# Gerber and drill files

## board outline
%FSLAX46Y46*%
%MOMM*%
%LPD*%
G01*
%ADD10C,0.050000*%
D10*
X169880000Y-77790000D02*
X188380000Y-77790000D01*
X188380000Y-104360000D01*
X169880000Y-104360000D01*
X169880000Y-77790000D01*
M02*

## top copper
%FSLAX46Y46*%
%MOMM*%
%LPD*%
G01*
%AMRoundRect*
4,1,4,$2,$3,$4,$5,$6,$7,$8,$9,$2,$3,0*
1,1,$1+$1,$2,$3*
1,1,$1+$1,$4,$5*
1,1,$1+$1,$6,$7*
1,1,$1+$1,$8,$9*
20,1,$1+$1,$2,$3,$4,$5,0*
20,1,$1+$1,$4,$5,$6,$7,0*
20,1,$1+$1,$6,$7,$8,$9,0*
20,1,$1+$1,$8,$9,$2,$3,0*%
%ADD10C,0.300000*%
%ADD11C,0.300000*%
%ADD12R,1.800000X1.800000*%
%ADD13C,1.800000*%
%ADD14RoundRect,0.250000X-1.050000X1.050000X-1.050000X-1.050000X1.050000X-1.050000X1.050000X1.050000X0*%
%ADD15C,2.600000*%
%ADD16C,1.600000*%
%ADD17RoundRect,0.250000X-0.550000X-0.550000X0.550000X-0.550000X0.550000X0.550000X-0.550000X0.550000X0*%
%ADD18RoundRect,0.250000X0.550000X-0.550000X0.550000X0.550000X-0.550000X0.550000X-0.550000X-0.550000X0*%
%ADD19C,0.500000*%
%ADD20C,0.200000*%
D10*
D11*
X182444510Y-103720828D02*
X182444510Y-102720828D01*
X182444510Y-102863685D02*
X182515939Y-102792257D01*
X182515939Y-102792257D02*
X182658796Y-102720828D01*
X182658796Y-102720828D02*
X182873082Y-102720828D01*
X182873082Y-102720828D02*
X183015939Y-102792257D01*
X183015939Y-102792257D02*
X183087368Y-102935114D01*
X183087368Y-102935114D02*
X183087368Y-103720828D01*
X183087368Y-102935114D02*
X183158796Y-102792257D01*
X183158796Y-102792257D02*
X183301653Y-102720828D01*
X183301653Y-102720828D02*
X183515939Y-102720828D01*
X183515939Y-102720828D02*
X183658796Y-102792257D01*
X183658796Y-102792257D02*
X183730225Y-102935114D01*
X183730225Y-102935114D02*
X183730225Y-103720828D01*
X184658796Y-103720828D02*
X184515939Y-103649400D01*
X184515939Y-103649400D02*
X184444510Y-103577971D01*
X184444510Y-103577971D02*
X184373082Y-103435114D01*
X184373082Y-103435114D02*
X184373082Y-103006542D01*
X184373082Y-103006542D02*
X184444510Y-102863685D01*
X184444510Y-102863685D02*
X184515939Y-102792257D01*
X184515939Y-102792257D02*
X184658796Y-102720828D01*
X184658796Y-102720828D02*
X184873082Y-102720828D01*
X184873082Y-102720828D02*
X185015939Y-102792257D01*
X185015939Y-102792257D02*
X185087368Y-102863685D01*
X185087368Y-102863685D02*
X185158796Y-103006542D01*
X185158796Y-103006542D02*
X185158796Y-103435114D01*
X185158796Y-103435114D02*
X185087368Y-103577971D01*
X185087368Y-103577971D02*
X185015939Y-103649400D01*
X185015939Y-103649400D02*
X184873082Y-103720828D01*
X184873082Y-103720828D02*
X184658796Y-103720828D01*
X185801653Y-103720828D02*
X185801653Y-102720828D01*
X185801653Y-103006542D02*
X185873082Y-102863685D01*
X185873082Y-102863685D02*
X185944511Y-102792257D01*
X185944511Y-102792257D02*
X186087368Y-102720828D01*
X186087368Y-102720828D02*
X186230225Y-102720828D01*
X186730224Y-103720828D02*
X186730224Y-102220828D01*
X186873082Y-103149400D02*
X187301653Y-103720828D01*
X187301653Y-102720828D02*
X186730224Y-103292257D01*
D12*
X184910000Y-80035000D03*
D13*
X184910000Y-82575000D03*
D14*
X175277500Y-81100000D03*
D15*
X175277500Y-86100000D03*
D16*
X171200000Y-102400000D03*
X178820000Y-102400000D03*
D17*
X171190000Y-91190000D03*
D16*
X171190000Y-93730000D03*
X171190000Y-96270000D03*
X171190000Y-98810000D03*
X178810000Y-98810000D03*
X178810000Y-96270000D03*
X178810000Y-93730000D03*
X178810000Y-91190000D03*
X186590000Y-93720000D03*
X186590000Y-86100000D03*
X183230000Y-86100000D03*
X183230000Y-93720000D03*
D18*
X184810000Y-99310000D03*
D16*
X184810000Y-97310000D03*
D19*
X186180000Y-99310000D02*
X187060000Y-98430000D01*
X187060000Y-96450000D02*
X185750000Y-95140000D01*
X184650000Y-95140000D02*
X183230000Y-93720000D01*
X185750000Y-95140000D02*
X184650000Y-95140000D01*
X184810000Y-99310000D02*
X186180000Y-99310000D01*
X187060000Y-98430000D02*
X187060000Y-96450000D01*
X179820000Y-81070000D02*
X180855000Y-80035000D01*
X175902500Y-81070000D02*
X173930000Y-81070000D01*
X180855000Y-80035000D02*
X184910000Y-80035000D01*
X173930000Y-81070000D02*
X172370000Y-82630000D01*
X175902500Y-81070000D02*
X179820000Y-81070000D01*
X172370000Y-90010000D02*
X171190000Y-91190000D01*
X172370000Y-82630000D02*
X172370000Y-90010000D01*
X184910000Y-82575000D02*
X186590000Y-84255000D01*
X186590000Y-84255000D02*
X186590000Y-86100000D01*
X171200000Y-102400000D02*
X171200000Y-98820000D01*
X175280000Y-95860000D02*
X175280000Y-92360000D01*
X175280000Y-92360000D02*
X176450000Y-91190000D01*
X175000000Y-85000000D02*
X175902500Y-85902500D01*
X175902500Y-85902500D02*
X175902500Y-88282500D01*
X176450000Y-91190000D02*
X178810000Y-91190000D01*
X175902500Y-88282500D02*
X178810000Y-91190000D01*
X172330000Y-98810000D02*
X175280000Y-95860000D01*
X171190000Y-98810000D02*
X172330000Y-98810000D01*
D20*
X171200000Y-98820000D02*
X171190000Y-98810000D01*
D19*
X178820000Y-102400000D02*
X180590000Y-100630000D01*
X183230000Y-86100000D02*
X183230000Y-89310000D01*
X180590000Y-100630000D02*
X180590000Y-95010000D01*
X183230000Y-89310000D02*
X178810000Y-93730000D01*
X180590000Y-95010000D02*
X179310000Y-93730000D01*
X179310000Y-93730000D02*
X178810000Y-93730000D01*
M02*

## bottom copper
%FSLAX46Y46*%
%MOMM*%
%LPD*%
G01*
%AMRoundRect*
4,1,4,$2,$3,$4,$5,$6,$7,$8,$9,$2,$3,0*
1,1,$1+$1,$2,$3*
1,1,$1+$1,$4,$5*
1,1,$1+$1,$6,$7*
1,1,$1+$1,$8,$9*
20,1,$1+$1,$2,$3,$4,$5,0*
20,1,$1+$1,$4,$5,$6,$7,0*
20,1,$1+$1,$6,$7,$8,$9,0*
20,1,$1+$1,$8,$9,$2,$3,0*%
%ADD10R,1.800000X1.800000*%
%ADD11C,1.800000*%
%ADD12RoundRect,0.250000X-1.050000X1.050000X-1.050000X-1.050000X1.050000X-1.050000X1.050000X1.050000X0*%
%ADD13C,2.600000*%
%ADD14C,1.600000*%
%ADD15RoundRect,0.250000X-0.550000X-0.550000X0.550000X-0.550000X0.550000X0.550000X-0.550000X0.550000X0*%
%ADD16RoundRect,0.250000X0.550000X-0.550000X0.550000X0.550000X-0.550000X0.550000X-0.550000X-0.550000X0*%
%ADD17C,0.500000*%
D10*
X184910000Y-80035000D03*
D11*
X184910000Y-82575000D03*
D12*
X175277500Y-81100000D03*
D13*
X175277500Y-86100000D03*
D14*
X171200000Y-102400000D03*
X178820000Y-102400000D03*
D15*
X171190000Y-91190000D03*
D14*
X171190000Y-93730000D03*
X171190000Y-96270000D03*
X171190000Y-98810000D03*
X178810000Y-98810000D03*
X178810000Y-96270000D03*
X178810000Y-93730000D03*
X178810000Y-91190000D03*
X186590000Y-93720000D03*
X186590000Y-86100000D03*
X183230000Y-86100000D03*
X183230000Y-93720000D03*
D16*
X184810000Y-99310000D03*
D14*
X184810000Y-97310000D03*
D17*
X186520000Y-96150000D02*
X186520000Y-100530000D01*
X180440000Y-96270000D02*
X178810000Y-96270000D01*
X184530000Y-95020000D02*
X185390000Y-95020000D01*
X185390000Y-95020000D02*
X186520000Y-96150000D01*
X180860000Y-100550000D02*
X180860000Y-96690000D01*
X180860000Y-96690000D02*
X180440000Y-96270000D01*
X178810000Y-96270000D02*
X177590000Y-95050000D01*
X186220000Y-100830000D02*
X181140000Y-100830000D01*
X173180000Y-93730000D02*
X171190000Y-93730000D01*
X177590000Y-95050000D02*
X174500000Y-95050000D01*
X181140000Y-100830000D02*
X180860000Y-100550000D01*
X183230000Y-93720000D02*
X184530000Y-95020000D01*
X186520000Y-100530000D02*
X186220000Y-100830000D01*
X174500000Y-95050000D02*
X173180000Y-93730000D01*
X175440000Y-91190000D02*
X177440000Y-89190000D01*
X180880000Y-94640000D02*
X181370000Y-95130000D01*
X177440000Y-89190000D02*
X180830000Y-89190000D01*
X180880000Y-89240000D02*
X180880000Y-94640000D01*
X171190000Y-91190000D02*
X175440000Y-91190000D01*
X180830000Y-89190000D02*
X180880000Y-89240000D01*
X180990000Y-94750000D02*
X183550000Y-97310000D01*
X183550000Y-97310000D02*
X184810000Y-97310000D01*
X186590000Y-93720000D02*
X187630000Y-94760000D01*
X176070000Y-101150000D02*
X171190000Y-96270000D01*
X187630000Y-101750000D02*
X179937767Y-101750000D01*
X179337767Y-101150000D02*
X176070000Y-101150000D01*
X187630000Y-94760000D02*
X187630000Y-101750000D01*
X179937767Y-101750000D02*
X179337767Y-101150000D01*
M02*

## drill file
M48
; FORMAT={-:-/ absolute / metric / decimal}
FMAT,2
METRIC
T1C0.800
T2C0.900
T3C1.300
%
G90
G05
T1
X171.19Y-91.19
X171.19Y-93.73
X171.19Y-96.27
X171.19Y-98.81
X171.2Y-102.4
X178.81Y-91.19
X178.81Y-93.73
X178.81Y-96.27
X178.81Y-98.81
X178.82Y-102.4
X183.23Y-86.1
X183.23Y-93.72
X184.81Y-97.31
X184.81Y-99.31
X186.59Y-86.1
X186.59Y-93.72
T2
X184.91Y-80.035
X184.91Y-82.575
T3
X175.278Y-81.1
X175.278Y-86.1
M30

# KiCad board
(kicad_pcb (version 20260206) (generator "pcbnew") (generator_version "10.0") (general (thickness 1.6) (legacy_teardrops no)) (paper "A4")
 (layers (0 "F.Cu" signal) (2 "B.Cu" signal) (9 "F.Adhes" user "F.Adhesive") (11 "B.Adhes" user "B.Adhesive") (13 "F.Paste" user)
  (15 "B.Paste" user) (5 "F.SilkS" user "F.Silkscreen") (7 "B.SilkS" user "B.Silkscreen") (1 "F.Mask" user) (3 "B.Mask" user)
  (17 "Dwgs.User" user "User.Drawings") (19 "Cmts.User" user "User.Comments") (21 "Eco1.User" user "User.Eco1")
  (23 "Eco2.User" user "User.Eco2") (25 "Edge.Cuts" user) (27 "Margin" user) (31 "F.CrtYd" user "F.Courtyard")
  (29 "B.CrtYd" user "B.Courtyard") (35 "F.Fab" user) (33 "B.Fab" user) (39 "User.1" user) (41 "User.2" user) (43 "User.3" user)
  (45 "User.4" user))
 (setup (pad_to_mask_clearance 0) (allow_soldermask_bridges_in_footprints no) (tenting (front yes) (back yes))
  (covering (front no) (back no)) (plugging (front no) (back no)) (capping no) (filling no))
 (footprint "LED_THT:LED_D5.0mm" (layer "F.Cu") (at 184.91 80.035 -90)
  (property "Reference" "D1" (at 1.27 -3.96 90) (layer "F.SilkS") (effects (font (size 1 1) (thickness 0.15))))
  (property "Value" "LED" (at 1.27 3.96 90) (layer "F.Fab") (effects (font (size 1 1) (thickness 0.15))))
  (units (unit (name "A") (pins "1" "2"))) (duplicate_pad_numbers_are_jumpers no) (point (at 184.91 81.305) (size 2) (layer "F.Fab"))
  (pad "1" thru_hole rect (at 0 0 270) (size 1.8 1.8) (drill 0.9) (layers "*.Cu" "*.Mask") (remove_unused_layers no) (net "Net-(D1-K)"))
  (pad "2" thru_hole circle (at 2.54 0 270) (size 1.8 1.8) (drill 0.9) (layers "*.Cu" "*.Mask") (remove_unused_layers no) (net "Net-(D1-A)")))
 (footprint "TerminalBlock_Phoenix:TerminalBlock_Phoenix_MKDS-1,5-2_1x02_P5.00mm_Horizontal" (layer "F.Cu") (at 175.2775 81.1 -90)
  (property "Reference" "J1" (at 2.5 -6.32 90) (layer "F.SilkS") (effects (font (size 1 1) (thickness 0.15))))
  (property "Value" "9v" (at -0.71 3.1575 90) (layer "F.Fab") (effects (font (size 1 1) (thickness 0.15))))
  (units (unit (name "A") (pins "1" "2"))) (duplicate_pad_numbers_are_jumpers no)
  (pad "1" thru_hole roundrect (at 0 0 270) (size 2.6 2.6) (drill 1.3) (layers "*.Cu" "*.Mask") (remove_unused_layers no)
   (roundrect_rratio 0.096154) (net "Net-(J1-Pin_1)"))
  (pad "2" thru_hole circle (at 5 0 270) (size 2.6 2.6) (drill 1.3) (layers "*.Cu" "*.Mask") (remove_unused_layers no) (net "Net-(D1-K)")))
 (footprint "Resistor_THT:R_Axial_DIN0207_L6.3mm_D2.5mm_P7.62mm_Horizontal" (layer "F.Cu") (at 171.2 102.4)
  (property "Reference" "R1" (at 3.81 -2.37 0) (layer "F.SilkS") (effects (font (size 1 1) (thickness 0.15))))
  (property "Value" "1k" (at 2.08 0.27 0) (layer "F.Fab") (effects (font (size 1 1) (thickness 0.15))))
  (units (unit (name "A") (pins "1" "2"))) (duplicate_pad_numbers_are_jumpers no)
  (pad "1" thru_hole circle (at 0 0) (size 1.6 1.6) (drill 0.8) (layers "*.Cu" "*.Mask") (remove_unused_layers no) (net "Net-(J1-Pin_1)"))
  (pad "2" thru_hole circle (at 7.62 0) (size 1.6 1.6) (drill 0.8) (layers "*.Cu" "*.Mask") (remove_unused_layers no) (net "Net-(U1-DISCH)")))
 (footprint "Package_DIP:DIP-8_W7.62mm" (layer "F.Cu") (at 171.19 91.19)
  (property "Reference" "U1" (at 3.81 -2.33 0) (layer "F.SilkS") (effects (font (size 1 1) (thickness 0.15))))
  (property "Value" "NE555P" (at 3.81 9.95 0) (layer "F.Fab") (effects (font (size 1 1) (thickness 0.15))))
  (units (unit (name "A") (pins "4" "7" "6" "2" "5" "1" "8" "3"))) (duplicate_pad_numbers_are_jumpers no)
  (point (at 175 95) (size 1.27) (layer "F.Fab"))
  (pad "1" thru_hole roundrect (at 0 0) (size 1.6 1.6) (drill 0.8) (layers "*.Cu" "*.Mask") (remove_unused_layers no)
   (roundrect_rratio 0.15625) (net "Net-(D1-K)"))
  (pad "2" thru_hole circle (at 0 2.54) (size 1.6 1.6) (drill 0.8) (layers "*.Cu" "*.Mask") (remove_unused_layers no) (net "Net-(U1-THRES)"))
  (pad "3" thru_hole circle (at 0 5.08) (size 1.6 1.6) (drill 0.8) (layers "*.Cu" "*.Mask") (remove_unused_layers no) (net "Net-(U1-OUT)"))
  (pad "4" thru_hole circle (at 0 7.62) (size 1.6 1.6) (drill 0.8) (layers "*.Cu" "*.Mask") (remove_unused_layers no) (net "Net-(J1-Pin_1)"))
  (pad "5" thru_hole circle (at 7.62 7.62) (size 1.6 1.6) (drill 0.8) (layers "*.Cu" "*.Mask") (remove_unused_layers no) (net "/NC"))
  (pad "6" thru_hole circle (at 7.62 5.08) (size 1.6 1.6) (drill 0.8) (layers "*.Cu" "*.Mask") (remove_unused_layers no)
   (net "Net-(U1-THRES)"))
  (pad "7" thru_hole circle (at 7.62 2.54) (size 1.6 1.6) (drill 0.8) (layers "*.Cu" "*.Mask") (remove_unused_layers no)
   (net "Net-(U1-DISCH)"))
  (pad "8" thru_hole circle (at 7.62 0) (size 1.6 1.6) (drill 0.8) (layers "*.Cu" "*.Mask") (remove_unused_layers no) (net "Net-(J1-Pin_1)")))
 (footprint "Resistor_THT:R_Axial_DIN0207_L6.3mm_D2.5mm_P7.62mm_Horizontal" (layer "F.Cu") (at 186.59 93.72 90)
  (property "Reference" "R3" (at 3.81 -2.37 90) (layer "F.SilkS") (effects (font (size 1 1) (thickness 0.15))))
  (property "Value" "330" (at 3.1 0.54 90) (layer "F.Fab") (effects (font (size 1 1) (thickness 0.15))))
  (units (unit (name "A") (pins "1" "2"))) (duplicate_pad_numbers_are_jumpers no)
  (pad "1" thru_hole circle (at 0 0 90) (size 1.6 1.6) (drill 0.8) (layers "*.Cu" "*.Mask") (remove_unused_layers no) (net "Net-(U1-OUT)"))
  (pad "2" thru_hole circle (at 7.62 0 90) (size 1.6 1.6) (drill 0.8) (layers "*.Cu" "*.Mask") (remove_unused_layers no) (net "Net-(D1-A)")))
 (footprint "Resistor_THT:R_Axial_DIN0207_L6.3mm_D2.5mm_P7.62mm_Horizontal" (layer "F.Cu") (at 183.23 86.1 -90)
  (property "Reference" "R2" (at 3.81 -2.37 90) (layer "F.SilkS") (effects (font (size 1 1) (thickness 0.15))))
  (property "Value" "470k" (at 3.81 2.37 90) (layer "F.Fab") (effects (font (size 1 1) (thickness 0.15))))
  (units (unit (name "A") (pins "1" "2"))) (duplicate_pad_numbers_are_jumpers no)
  (pad "1" thru_hole circle (at 0 0 270) (size 1.6 1.6) (drill 0.8) (layers "*.Cu" "*.Mask") (remove_unused_layers no)
   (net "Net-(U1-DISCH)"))
  (pad "2" thru_hole circle (at 7.62 0 270) (size 1.6 1.6) (drill 0.8) (layers "*.Cu" "*.Mask") (remove_unused_layers no)
   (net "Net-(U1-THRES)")))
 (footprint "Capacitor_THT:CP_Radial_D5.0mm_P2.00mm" (layer "F.Cu") (at 184.81 99.31 90)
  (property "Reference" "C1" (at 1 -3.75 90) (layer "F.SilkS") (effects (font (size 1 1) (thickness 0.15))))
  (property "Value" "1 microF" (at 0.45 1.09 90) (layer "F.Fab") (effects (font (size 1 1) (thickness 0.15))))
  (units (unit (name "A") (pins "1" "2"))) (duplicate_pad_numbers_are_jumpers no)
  (pad "1" thru_hole roundrect (at 0 0 90) (size 1.6 1.6) (drill 0.8) (layers "*.Cu" "*.Mask") (remove_unused_layers no)
   (roundrect_rratio 0.15625) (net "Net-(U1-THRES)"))
  (pad "2" thru_hole circle (at 2 0 90) (size 1.6 1.6) (drill 0.8) (layers "*.Cu" "*.Mask") (remove_unused_layers no) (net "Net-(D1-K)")))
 (gr_rect (start 169.88 77.79) (end 188.38 104.36) (stroke (width 0.05) (type default)) (fill no) (layer "Edge.Cuts"))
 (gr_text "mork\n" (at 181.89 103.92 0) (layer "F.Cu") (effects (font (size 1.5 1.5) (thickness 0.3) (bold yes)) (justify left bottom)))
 (segment (start 186.18 99.31) (end 187.06 98.43) (width 0.5) (layer "F.Cu") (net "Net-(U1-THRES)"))
 (segment (start 187.06 96.45) (end 185.75 95.14) (width 0.5) (layer "F.Cu") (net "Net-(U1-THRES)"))
 (segment (start 184.65 95.14) (end 183.23 93.72) (width 0.5) (layer "F.Cu") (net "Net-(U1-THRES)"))
 (segment (start 185.75 95.14) (end 184.65 95.14) (width 0.5) (layer "F.Cu") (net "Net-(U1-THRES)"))
 (segment (start 184.81 99.31) (end 186.18 99.31) (width 0.5) (layer "F.Cu") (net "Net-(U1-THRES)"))
 (segment (start 187.06 98.43) (end 187.06 96.45) (width 0.5) (layer "F.Cu") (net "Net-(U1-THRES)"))
 (segment (start 186.52 96.15) (end 186.52 100.53) (width 0.5) (layer "B.Cu") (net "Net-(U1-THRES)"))
 (segment (start 180.44 96.27) (end 178.81 96.27) (width 0.5) (layer "B.Cu") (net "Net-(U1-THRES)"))
 (segment (start 184.53 95.02) (end 185.39 95.02) (width 0.5) (layer "B.Cu") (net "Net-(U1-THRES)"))
 (segment (start 185.39 95.02) (end 186.52 96.15) (width 0.5) (layer "B.Cu") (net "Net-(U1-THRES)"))
 (segment (start 180.86 100.55) (end 180.86 96.69) (width 0.5) (layer "B.Cu") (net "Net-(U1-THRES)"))
 (segment (start 180.86 96.69) (end 180.44 96.27) (width 0.5) (layer "B.Cu") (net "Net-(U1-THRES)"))
 (segment (start 178.81 96.27) (end 177.59 95.05) (width 0.5) (layer "B.Cu") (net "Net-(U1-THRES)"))
 (segment (start 186.22 100.83) (end 181.14 100.83) (width 0.5) (layer "B.Cu") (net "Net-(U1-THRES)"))
 (segment (start 173.18 93.73) (end 171.19 93.73) (width 0.5) (layer "B.Cu") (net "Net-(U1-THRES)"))
 (segment (start 177.59 95.05) (end 174.5 95.05) (width 0.5) (layer "B.Cu") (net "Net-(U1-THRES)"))
 (segment (start 181.14 100.83) (end 180.86 100.55) (width 0.5) (layer "B.Cu") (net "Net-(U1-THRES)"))
 (segment (start 183.23 93.72) (end 184.53 95.02) (width 0.5) (layer "B.Cu") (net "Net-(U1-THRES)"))
 (segment (start 186.52 100.53) (end 186.22 100.83) (width 0.5) (layer "B.Cu") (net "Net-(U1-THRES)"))
 (segment (start 174.5 95.05) (end 173.18 93.73) (width 0.5) (layer "B.Cu") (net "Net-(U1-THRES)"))
 (segment (start 179.82 81.07) (end 180.855 80.035) (width 0.5) (layer "F.Cu") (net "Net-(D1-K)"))
 (segment (start 175.9025 81.07) (end 173.93 81.07) (width 0.5) (layer "F.Cu") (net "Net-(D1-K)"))
 (segment (start 180.855 80.035) (end 184.91 80.035) (width 0.5) (layer "F.Cu") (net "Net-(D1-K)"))
 (segment (start 173.93 81.07) (end 172.37 82.63) (width 0.5) (layer "F.Cu") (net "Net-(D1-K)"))
 (segment (start 175.9025 81.07) (end 179.82 81.07) (width 0.5) (layer "F.Cu") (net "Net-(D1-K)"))
 (segment (start 172.37 90.01) (end 171.19 91.19) (width 0.5) (layer "F.Cu") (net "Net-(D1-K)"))
 (segment (start 172.37 82.63) (end 172.37 90.01) (width 0.5) (layer "F.Cu") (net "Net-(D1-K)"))
 (segment (start 175.44 91.19) (end 177.44 89.19) (width 0.5) (layer "B.Cu") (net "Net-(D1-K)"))
 (segment (start 180.88 94.64) (end 181.37 95.13) (width 0.5) (layer "B.Cu") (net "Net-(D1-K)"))
 (segment (start 177.44 89.19) (end 180.83 89.19) (width 0.5) (layer "B.Cu") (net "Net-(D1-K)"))
 (segment (start 180.88 89.24) (end 180.88 94.64) (width 0.5) (layer "B.Cu") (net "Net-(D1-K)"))
 (segment (start 171.19 91.19) (end 175.44 91.19) (width 0.5) (layer "B.Cu") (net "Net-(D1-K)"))
 (segment (start 180.83 89.19) (end 180.88 89.24) (width 0.5) (layer "B.Cu") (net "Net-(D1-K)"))
 (segment (start 180.99 94.75) (end 183.55 97.31) (width 0.5) (layer "B.Cu") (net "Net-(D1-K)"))
 (segment (start 183.55 97.31) (end 184.81 97.31) (width 0.5) (layer "B.Cu") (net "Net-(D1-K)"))
 (segment (start 184.91 82.575) (end 186.59 84.255) (width 0.5) (layer "F.Cu") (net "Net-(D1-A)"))
 (segment (start 186.59 84.255) (end 186.59 86.1) (width 0.5) (layer "F.Cu") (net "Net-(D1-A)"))
 (segment (start 171.2 102.4) (end 171.2 98.82) (width 0.5) (layer "F.Cu") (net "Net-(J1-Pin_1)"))
 (segment (start 175.28 95.86) (end 175.28 92.36) (width 0.5) (layer "F.Cu") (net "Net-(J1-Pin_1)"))
 (segment (start 175.28 92.36) (end 176.45 91.19) (width 0.5) (layer "F.Cu") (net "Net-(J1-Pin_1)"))
 (segment (start 175 85) (end 175.9025 85.9025) (width 0.5) (layer "F.Cu") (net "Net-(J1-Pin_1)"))
 (segment (start 175.9025 85.9025) (end 175.9025 88.2825) (width 0.5) (layer "F.Cu") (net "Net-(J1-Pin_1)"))
 (segment (start 176.45 91.19) (end 178.81 91.19) (width 0.5) (layer "F.Cu") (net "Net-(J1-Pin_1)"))
 (segment (start 175.9025 88.2825) (end 178.81 91.19) (width 0.5) (layer "F.Cu") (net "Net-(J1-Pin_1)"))
 (segment (start 172.33 98.81) (end 175.28 95.86) (width 0.5) (layer "F.Cu") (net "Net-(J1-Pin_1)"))
 (segment (start 171.19 98.81) (end 172.33 98.81) (width 0.5) (layer "F.Cu") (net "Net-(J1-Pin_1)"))
 (segment (start 171.2 98.82) (end 171.19 98.81) (width 0.2) (layer "F.Cu") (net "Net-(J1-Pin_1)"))
 (segment (start 178.82 102.4) (end 180.59 100.63) (width 0.5) (layer "F.Cu") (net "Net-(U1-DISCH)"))
 (segment (start 183.23 86.1) (end 183.23 89.31) (width 0.5) (layer "F.Cu") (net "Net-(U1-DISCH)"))
 (segment (start 180.59 100.63) (end 180.59 95.01) (width 0.5) (layer "F.Cu") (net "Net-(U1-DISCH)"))
 (segment (start 183.23 89.31) (end 178.81 93.73) (width 0.5) (layer "F.Cu") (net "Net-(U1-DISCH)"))
 (segment (start 180.59 95.01) (end 179.31 93.73) (width 0.5) (layer "F.Cu") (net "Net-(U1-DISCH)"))
 (segment (start 179.31 93.73) (end 178.81 93.73) (width 0.5) (layer "F.Cu") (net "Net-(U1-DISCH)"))
 (segment (start 186.59 93.72) (end 187.63 94.76) (width 0.5) (layer "B.Cu") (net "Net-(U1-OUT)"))
 (segment (start 176.07 101.15) (end 171.19 96.27) (width 0.5) (layer "B.Cu") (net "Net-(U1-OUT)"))
 (segment (start 187.63 101.75) (end 179.937767 101.75) (width 0.5) (layer "B.Cu") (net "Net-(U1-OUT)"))
 (segment (start 179.337767 101.15) (end 176.07 101.15) (width 0.5) (layer "B.Cu") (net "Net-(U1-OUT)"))
 (segment (start 187.63 94.76) (end 187.63 101.75) (width 0.5) (layer "B.Cu") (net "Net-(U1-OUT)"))
 (segment (start 179.937767 101.75) (end 179.337767 101.15) (width 0.5) (layer "B.Cu") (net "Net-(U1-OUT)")))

